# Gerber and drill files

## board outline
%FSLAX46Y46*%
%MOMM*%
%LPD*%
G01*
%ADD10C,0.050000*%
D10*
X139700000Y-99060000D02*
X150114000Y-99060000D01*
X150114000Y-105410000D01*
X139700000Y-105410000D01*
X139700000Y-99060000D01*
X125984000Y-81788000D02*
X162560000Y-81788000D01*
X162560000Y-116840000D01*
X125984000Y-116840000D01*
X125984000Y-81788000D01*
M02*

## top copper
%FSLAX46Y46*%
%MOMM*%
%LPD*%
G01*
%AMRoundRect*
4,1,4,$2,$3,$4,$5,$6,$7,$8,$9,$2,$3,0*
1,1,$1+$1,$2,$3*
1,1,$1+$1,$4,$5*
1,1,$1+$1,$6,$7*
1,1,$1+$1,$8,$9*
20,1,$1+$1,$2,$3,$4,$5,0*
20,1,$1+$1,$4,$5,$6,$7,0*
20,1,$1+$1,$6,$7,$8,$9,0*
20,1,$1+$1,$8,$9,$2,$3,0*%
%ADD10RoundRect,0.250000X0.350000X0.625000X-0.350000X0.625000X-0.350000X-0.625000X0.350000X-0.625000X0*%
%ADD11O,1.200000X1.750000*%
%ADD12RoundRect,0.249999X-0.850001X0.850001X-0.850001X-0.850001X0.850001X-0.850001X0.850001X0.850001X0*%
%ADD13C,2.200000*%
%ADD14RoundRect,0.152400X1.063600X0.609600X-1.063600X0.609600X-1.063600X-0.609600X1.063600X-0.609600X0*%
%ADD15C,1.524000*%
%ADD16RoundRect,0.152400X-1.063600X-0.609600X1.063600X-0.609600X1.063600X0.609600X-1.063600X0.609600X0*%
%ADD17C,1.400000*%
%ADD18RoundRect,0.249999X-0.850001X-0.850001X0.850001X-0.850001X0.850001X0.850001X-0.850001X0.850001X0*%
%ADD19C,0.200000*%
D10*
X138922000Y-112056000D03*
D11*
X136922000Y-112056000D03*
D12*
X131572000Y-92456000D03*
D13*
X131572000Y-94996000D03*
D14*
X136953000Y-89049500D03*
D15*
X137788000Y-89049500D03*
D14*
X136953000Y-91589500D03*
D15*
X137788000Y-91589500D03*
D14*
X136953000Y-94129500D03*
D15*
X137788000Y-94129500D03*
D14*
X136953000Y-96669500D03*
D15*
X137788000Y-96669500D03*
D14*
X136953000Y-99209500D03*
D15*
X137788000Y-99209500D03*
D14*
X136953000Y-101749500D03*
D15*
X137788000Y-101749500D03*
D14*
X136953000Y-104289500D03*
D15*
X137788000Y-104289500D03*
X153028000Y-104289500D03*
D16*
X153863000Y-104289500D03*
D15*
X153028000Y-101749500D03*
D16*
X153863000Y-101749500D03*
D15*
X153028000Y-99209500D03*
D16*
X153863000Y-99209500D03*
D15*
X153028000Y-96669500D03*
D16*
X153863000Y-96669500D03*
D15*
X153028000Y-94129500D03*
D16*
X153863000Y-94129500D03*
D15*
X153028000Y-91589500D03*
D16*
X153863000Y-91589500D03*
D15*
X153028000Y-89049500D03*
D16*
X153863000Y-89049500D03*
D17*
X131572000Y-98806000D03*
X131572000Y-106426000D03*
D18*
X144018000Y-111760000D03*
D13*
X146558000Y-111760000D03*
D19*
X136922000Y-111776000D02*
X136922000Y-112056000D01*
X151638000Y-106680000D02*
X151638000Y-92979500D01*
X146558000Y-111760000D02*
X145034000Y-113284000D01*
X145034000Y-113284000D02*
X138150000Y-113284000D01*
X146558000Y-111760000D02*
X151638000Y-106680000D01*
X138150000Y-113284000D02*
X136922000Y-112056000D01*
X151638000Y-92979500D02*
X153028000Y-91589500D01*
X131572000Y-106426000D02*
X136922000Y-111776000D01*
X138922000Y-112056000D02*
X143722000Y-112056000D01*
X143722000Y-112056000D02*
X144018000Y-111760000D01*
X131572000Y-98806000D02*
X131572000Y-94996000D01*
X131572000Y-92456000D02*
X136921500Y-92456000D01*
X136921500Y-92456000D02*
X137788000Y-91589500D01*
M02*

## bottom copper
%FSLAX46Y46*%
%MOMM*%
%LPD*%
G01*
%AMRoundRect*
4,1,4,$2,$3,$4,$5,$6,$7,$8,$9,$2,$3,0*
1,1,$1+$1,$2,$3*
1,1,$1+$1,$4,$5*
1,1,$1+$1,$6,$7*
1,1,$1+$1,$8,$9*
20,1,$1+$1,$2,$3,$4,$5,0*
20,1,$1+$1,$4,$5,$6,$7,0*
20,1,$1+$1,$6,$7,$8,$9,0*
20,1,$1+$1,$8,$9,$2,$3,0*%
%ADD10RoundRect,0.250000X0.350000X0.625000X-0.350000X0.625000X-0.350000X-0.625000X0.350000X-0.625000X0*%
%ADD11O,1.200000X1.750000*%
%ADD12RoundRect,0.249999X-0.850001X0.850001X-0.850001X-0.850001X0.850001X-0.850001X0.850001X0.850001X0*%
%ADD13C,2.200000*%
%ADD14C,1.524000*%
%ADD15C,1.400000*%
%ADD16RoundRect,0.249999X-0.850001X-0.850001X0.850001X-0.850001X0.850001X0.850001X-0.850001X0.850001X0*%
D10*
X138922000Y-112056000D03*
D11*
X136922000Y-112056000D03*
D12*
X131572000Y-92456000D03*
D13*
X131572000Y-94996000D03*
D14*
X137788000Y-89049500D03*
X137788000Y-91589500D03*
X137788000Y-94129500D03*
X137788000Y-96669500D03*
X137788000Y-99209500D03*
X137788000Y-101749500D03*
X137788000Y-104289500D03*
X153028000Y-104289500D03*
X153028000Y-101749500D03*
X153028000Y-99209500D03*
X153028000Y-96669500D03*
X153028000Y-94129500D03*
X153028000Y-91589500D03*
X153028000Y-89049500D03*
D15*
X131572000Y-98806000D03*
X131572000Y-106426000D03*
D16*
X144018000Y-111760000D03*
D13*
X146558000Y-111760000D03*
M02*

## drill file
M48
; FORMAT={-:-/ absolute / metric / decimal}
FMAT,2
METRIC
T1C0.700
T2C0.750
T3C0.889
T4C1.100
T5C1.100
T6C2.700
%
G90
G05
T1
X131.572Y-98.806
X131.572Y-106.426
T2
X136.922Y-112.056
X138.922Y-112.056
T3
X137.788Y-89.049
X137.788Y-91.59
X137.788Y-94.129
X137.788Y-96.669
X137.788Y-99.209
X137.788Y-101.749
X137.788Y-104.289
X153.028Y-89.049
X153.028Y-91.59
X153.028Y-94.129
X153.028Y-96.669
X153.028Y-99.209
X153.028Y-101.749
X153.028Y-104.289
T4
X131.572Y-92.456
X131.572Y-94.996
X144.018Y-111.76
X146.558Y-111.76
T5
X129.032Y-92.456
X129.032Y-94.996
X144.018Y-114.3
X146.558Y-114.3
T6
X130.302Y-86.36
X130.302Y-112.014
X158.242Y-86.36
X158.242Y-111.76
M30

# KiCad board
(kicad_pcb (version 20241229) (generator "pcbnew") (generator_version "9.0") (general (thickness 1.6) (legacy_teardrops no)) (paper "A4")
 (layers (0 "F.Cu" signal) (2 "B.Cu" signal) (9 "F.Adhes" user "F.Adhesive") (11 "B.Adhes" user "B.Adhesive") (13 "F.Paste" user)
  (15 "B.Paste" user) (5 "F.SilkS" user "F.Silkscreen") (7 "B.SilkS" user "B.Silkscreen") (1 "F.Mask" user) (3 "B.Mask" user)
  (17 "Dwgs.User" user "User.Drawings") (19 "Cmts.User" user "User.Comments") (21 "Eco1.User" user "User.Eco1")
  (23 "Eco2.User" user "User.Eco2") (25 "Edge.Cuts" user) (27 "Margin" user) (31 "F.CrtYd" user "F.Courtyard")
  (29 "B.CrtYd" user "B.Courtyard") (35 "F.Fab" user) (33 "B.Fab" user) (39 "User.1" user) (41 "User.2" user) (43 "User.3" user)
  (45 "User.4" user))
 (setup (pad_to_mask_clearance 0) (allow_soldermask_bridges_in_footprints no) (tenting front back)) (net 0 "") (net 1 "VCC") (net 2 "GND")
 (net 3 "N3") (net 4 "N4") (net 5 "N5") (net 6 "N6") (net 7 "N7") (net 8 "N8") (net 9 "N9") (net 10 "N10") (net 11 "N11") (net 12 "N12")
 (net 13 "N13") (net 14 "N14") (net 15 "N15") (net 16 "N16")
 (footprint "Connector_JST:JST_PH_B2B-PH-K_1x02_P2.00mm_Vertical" (layer "F.Cu") (at 138.922 112.056 180)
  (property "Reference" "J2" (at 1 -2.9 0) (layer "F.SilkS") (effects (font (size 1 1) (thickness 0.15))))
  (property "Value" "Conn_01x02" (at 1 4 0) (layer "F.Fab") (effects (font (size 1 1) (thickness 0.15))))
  (pad "1" thru_hole roundrect (at 0 0 180) (size 1.2 1.75) (drill 0.75) (layers "*.Cu" "*.Mask") (remove_unused_layers no)
   (roundrect_rratio 0.208333) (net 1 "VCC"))
  (pad "2" thru_hole oval (at 2 0 180) (size 1.2 1.75) (drill 0.75) (layers "*.Cu" "*.Mask") (remove_unused_layers no) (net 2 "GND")))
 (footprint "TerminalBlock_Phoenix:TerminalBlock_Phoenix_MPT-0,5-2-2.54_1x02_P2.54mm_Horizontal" (layer "F.Cu") (at 131.572 92.456 -90)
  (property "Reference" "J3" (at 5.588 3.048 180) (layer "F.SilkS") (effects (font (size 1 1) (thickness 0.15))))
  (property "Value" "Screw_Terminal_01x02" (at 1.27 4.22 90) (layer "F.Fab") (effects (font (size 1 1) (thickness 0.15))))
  (pad "" np_thru_hole circle (at 0 2.54 270) (size 1.1 1.1) (drill 1.1) (layers "*.Cu" "*.Mask"))
  (pad "" np_thru_hole circle (at 2.54 2.54 270) (size 1.1 1.1) (drill 1.1) (layers "*.Cu" "*.Mask"))
  (pad "1" thru_hole roundrect (at 0 0 270) (size 2.2 2.2) (drill 1.1) (layers "*.Cu" "*.Mask") (remove_unused_layers no)
   (roundrect_rratio 0.113636) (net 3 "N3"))
  (pad "2" thru_hole circle (at 2.54 0 270) (size 2.2 2.2) (drill 1.1) (layers "*.Cu" "*.Mask") (remove_unused_layers no) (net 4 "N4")))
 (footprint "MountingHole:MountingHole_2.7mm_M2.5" (layer "F.Cu") (at 130.302 112.014)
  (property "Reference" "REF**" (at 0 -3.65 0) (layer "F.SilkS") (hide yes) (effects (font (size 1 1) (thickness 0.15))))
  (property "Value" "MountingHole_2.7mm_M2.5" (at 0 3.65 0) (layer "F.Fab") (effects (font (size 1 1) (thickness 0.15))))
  (pad "" np_thru_hole circle (at 0 0) (size 2.7 2.7) (drill 2.7) (layers "*.Cu" "*.Mask")))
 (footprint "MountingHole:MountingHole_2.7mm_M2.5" (layer "F.Cu") (at 130.302 86.36)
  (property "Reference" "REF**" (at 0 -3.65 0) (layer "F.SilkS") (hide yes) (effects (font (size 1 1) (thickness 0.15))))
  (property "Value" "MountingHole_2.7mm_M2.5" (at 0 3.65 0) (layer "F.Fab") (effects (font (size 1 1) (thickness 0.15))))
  (pad "" np_thru_hole circle (at 0 0) (size 2.7 2.7) (drill 2.7) (layers "*.Cu" "*.Mask")))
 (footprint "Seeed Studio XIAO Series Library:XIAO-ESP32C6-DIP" (layer "F.Cu") (at 145.453 96.6695)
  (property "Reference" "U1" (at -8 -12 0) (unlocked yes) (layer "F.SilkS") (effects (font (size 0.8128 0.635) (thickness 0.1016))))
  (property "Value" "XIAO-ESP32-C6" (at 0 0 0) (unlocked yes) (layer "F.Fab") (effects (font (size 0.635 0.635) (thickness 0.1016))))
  (pad "1" smd roundrect (at -8.5 -7.62 180) (size 2.432 1.524) (layers "F.Cu" "F.Mask") (roundrect_rratio 0.1) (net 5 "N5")
   (thermal_bridge_angle 45))
  (pad "1" thru_hole circle (at -7.665 -7.62 180) (size 1.524 1.524) (drill 0.889) (layers "*.Cu" "*.Mask") (remove_unused_layers no)
   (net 5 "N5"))
  (pad "2" smd roundrect (at -8.5 -5.08 180) (size 2.432 1.524) (layers "F.Cu" "F.Mask") (roundrect_rratio 0.1) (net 3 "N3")
   (thermal_bridge_angle 45))
  (pad "2" thru_hole circle (at -7.665 -5.08 180) (size 1.524 1.524) (drill 0.889) (layers "*.Cu" "*.Mask") (remove_unused_layers no)
   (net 3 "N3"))
  (pad "3" smd roundrect (at -8.5 -2.54 180) (size 2.432 1.524) (layers "F.Cu" "F.Mask") (roundrect_rratio 0.1) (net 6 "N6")
   (thermal_bridge_angle 45))
  (pad "3" thru_hole circle (at -7.665 -2.54 180) (size 1.524 1.524) (drill 0.889) (layers "*.Cu" "*.Mask") (remove_unused_layers no)
   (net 6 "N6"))
  (pad "4" smd roundrect (at -8.5 0 180) (size 2.432 1.524) (layers "F.Cu" "F.Mask") (roundrect_rratio 0.1) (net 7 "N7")
   (thermal_bridge_angle 45))
  (pad "4" thru_hole circle (at -7.665 0 180) (size 1.524 1.524) (drill 0.889) (layers "*.Cu" "*.Mask") (remove_unused_layers no)
   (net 7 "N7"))
  (pad "5" smd roundrect (at -8.5 2.54 180) (size 2.432 1.524) (layers "F.Cu" "F.Mask") (roundrect_rratio 0.1) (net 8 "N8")
   (thermal_bridge_angle 45))
  (pad "5" thru_hole circle (at -7.665 2.54 180) (size 1.524 1.524) (drill 0.889) (layers "*.Cu" "*.Mask") (remove_unused_layers no)
   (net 8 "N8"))
  (pad "6" smd roundrect (at -8.5 5.08 180) (size 2.432 1.524) (layers "F.Cu" "F.Mask") (roundrect_rratio 0.1) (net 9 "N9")
   (thermal_bridge_angle 45))
  (pad "6" thru_hole circle (at -7.665 5.08 180) (size 1.524 1.524) (drill 0.889) (layers "*.Cu" "*.Mask") (remove_unused_layers no)
   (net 9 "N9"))
  (pad "7" smd roundrect (at -8.5 7.62 180) (size 2.432 1.524) (layers "F.Cu" "F.Mask") (roundrect_rratio 0.1) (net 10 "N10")
   (thermal_bridge_angle 45))
  (pad "7" thru_hole circle (at -7.665 7.62 180) (size 1.524 1.524) (drill 0.889) (layers "*.Cu" "*.Mask") (remove_unused_layers no)
   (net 10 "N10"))
  (pad "8" thru_hole circle (at 7.575 7.62) (size 1.524 1.524) (drill 0.889) (layers "*.Cu" "*.Mask") (remove_unused_layers no)
   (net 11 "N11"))
  (pad "8" smd roundrect (at 8.41 7.62) (size 2.432 1.524) (layers "F.Cu" "F.Mask") (roundrect_rratio 0.1) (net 11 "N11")
   (thermal_bridge_angle 45))
  (pad "9" thru_hole circle (at 7.575 5.08) (size 1.524 1.524) (drill 0.889) (layers "*.Cu" "*.Mask") (remove_unused_layers no)
   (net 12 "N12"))
  (pad "9" smd roundrect (at 8.41 5.08) (size 2.432 1.524) (layers "F.Cu" "F.Mask") (roundrect_rratio 0.1) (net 12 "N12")
   (thermal_bridge_angle 45))
  (pad "10" thru_hole circle (at 7.575 2.54) (size 1.524 1.524) (drill 0.889) (layers "*.Cu" "*.Mask") (remove_unused_layers no)
   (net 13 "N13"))
  (pad "10" smd roundrect (at 8.41 2.54) (size 2.432 1.524) (layers "F.Cu" "F.Mask") (roundrect_rratio 0.1) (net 13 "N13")
   (thermal_bridge_angle 45))
  (pad "11" thru_hole circle (at 7.575 0) (size 1.524 1.524) (drill 0.889) (layers "*.Cu" "*.Mask") (remove_unused_layers no) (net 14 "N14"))
  (pad "11" smd roundrect (at 8.41 0) (size 2.432 1.524) (layers "F.Cu" "F.Mask") (roundrect_rratio 0.1) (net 14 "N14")
   (thermal_bridge_angle 45))
  (pad "12" thru_hole circle (at 7.575 -2.54) (size 1.524 1.524) (drill 0.889) (layers "*.Cu" "*.Mask") (remove_unused_layers no)
   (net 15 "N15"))
  (pad "12" smd roundrect (at 8.41 -2.54) (size 2.432 1.524) (layers "F.Cu" "F.Mask") (roundrect_rratio 0.1) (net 15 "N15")
   (thermal_bridge_angle 45))
  (pad "13" thru_hole circle (at 7.575 -5.08) (size 1.524 1.524) (drill 0.889) (layers "*.Cu" "*.Mask") (remove_unused_layers no)
   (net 2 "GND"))
  (pad "13" smd roundrect (at 8.41 -5.08) (size 2.432 1.524) (layers "F.Cu" "F.Mask") (roundrect_rratio 0.1) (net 2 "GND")
   (thermal_bridge_angle 45))
  (pad "14" thru_hole circle (at 7.575 -7.62) (size 1.524 1.524) (drill 0.889) (layers "*.Cu" "*.Mask") (remove_unused_layers no)
   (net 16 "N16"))
  (pad "14" smd roundrect (at 8.41 -7.62) (size 2.432 1.524) (layers "F.Cu" "F.Mask") (roundrect_rratio 0.1) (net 16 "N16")
   (thermal_bridge_angle 45)))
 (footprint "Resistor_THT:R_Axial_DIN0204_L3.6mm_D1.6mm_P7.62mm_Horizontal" (layer "F.Cu") (at 131.572 98.806 -90)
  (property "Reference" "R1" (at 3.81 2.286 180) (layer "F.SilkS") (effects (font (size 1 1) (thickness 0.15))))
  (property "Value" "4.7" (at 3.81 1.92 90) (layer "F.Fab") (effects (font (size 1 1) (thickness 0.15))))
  (pad "1" thru_hole circle (at 0 0 270) (size 1.4 1.4) (drill 0.7) (layers "*.Cu" "*.Mask") (remove_unused_layers no) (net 4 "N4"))
  (pad "2" thru_hole circle (at 7.62 0 270) (size 1.4 1.4) (drill 0.7) (layers "*.Cu" "*.Mask") (remove_unused_layers no) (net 2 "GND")))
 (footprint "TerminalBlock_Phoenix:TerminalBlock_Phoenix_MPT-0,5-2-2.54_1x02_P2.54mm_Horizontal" (layer "F.Cu") (at 144.018 111.76)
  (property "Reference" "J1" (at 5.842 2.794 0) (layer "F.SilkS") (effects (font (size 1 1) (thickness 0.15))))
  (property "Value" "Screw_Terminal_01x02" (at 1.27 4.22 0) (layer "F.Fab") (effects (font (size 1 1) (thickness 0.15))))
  (pad "" np_thru_hole circle (at 0 2.54) (size 1.1 1.1) (drill 1.1) (layers "*.Cu" "*.Mask"))
  (pad "" np_thru_hole circle (at 2.54 2.54) (size 1.1 1.1) (drill 1.1) (layers "*.Cu" "*.Mask"))
  (pad "1" thru_hole roundrect (at 0 0) (size 2.2 2.2) (drill 1.1) (layers "*.Cu" "*.Mask") (remove_unused_layers no)
   (roundrect_rratio 0.113636) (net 1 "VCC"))
  (pad "2" thru_hole circle (at 2.54 0) (size 2.2 2.2) (drill 1.1) (layers "*.Cu" "*.Mask") (remove_unused_layers no) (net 2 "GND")))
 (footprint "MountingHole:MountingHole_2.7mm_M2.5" (layer "F.Cu") (at 158.242 111.76)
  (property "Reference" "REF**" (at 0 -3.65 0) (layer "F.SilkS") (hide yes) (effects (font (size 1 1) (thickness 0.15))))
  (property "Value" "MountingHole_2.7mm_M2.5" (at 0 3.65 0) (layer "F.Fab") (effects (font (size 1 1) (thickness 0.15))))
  (pad "" np_thru_hole circle (at 0 0) (size 2.7 2.7) (drill 2.7) (layers "*.Cu" "*.Mask")))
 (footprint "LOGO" (layer "F.Cu") (at 159.004 98.806)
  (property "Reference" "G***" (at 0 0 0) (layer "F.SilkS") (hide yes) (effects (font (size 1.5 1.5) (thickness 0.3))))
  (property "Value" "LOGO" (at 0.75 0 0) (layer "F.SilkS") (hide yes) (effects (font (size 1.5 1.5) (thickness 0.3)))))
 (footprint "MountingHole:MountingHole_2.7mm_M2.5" (layer "F.Cu") (at 158.242 86.36)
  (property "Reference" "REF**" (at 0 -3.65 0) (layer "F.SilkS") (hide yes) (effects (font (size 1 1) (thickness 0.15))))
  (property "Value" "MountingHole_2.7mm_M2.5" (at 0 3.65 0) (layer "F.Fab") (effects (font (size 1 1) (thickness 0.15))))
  (pad "" np_thru_hole circle (at 0 0) (size 2.7 2.7) (drill 2.7) (layers "*.Cu" "*.Mask")))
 (gr_rect (start 139.7 99.06) (end 150.114 105.41) (stroke (width 0.05) (type default)) (fill no) (layer "Edge.Cuts"))
 (gr_rect (start 125.984 81.788) (end 162.56 116.84) (stroke (width 0.05) (type default)) (fill no) (layer "Edge.Cuts"))
 (segment (start 136.922 111.776) (end 136.922 112.056) (width 0.2) (layer "F.Cu") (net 2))
 (segment (start 151.638 106.68) (end 151.638 92.9795) (width 0.2) (layer "F.Cu") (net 2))
 (segment (start 146.558 111.76) (end 145.034 113.284) (width 0.2) (layer "F.Cu") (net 2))
 (segment (start 145.034 113.284) (end 138.15 113.284) (width 0.2) (layer "F.Cu") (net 2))
 (segment (start 146.558 111.76) (end 151.638 106.68) (width 0.2) (layer "F.Cu") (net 2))
 (segment (start 138.15 113.284) (end 136.922 112.056) (width 0.2) (layer "F.Cu") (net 2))
 (segment (start 151.638 92.9795) (end 153.028 91.5895) (width 0.2) (layer "F.Cu") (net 2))
 (segment (start 131.572 106.426) (end 136.922 111.776) (width 0.2) (layer "F.Cu") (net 2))
 (segment (start 138.922 112.056) (end 143.722 112.056) (width 0.2) (layer "F.Cu") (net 1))
 (segment (start 143.722 112.056) (end 144.018 111.76) (width 0.2) (layer "F.Cu") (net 1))
 (segment (start 131.572 98.806) (end 131.572 94.996) (width 0.2) (layer "F.Cu") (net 4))
 (segment (start 131.572 92.456) (end 136.9215 92.456) (width 0.2) (layer "F.Cu") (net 3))
 (segment (start 136.9215 92.456) (end 137.788 91.5895) (width 0.2) (layer "F.Cu") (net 3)))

